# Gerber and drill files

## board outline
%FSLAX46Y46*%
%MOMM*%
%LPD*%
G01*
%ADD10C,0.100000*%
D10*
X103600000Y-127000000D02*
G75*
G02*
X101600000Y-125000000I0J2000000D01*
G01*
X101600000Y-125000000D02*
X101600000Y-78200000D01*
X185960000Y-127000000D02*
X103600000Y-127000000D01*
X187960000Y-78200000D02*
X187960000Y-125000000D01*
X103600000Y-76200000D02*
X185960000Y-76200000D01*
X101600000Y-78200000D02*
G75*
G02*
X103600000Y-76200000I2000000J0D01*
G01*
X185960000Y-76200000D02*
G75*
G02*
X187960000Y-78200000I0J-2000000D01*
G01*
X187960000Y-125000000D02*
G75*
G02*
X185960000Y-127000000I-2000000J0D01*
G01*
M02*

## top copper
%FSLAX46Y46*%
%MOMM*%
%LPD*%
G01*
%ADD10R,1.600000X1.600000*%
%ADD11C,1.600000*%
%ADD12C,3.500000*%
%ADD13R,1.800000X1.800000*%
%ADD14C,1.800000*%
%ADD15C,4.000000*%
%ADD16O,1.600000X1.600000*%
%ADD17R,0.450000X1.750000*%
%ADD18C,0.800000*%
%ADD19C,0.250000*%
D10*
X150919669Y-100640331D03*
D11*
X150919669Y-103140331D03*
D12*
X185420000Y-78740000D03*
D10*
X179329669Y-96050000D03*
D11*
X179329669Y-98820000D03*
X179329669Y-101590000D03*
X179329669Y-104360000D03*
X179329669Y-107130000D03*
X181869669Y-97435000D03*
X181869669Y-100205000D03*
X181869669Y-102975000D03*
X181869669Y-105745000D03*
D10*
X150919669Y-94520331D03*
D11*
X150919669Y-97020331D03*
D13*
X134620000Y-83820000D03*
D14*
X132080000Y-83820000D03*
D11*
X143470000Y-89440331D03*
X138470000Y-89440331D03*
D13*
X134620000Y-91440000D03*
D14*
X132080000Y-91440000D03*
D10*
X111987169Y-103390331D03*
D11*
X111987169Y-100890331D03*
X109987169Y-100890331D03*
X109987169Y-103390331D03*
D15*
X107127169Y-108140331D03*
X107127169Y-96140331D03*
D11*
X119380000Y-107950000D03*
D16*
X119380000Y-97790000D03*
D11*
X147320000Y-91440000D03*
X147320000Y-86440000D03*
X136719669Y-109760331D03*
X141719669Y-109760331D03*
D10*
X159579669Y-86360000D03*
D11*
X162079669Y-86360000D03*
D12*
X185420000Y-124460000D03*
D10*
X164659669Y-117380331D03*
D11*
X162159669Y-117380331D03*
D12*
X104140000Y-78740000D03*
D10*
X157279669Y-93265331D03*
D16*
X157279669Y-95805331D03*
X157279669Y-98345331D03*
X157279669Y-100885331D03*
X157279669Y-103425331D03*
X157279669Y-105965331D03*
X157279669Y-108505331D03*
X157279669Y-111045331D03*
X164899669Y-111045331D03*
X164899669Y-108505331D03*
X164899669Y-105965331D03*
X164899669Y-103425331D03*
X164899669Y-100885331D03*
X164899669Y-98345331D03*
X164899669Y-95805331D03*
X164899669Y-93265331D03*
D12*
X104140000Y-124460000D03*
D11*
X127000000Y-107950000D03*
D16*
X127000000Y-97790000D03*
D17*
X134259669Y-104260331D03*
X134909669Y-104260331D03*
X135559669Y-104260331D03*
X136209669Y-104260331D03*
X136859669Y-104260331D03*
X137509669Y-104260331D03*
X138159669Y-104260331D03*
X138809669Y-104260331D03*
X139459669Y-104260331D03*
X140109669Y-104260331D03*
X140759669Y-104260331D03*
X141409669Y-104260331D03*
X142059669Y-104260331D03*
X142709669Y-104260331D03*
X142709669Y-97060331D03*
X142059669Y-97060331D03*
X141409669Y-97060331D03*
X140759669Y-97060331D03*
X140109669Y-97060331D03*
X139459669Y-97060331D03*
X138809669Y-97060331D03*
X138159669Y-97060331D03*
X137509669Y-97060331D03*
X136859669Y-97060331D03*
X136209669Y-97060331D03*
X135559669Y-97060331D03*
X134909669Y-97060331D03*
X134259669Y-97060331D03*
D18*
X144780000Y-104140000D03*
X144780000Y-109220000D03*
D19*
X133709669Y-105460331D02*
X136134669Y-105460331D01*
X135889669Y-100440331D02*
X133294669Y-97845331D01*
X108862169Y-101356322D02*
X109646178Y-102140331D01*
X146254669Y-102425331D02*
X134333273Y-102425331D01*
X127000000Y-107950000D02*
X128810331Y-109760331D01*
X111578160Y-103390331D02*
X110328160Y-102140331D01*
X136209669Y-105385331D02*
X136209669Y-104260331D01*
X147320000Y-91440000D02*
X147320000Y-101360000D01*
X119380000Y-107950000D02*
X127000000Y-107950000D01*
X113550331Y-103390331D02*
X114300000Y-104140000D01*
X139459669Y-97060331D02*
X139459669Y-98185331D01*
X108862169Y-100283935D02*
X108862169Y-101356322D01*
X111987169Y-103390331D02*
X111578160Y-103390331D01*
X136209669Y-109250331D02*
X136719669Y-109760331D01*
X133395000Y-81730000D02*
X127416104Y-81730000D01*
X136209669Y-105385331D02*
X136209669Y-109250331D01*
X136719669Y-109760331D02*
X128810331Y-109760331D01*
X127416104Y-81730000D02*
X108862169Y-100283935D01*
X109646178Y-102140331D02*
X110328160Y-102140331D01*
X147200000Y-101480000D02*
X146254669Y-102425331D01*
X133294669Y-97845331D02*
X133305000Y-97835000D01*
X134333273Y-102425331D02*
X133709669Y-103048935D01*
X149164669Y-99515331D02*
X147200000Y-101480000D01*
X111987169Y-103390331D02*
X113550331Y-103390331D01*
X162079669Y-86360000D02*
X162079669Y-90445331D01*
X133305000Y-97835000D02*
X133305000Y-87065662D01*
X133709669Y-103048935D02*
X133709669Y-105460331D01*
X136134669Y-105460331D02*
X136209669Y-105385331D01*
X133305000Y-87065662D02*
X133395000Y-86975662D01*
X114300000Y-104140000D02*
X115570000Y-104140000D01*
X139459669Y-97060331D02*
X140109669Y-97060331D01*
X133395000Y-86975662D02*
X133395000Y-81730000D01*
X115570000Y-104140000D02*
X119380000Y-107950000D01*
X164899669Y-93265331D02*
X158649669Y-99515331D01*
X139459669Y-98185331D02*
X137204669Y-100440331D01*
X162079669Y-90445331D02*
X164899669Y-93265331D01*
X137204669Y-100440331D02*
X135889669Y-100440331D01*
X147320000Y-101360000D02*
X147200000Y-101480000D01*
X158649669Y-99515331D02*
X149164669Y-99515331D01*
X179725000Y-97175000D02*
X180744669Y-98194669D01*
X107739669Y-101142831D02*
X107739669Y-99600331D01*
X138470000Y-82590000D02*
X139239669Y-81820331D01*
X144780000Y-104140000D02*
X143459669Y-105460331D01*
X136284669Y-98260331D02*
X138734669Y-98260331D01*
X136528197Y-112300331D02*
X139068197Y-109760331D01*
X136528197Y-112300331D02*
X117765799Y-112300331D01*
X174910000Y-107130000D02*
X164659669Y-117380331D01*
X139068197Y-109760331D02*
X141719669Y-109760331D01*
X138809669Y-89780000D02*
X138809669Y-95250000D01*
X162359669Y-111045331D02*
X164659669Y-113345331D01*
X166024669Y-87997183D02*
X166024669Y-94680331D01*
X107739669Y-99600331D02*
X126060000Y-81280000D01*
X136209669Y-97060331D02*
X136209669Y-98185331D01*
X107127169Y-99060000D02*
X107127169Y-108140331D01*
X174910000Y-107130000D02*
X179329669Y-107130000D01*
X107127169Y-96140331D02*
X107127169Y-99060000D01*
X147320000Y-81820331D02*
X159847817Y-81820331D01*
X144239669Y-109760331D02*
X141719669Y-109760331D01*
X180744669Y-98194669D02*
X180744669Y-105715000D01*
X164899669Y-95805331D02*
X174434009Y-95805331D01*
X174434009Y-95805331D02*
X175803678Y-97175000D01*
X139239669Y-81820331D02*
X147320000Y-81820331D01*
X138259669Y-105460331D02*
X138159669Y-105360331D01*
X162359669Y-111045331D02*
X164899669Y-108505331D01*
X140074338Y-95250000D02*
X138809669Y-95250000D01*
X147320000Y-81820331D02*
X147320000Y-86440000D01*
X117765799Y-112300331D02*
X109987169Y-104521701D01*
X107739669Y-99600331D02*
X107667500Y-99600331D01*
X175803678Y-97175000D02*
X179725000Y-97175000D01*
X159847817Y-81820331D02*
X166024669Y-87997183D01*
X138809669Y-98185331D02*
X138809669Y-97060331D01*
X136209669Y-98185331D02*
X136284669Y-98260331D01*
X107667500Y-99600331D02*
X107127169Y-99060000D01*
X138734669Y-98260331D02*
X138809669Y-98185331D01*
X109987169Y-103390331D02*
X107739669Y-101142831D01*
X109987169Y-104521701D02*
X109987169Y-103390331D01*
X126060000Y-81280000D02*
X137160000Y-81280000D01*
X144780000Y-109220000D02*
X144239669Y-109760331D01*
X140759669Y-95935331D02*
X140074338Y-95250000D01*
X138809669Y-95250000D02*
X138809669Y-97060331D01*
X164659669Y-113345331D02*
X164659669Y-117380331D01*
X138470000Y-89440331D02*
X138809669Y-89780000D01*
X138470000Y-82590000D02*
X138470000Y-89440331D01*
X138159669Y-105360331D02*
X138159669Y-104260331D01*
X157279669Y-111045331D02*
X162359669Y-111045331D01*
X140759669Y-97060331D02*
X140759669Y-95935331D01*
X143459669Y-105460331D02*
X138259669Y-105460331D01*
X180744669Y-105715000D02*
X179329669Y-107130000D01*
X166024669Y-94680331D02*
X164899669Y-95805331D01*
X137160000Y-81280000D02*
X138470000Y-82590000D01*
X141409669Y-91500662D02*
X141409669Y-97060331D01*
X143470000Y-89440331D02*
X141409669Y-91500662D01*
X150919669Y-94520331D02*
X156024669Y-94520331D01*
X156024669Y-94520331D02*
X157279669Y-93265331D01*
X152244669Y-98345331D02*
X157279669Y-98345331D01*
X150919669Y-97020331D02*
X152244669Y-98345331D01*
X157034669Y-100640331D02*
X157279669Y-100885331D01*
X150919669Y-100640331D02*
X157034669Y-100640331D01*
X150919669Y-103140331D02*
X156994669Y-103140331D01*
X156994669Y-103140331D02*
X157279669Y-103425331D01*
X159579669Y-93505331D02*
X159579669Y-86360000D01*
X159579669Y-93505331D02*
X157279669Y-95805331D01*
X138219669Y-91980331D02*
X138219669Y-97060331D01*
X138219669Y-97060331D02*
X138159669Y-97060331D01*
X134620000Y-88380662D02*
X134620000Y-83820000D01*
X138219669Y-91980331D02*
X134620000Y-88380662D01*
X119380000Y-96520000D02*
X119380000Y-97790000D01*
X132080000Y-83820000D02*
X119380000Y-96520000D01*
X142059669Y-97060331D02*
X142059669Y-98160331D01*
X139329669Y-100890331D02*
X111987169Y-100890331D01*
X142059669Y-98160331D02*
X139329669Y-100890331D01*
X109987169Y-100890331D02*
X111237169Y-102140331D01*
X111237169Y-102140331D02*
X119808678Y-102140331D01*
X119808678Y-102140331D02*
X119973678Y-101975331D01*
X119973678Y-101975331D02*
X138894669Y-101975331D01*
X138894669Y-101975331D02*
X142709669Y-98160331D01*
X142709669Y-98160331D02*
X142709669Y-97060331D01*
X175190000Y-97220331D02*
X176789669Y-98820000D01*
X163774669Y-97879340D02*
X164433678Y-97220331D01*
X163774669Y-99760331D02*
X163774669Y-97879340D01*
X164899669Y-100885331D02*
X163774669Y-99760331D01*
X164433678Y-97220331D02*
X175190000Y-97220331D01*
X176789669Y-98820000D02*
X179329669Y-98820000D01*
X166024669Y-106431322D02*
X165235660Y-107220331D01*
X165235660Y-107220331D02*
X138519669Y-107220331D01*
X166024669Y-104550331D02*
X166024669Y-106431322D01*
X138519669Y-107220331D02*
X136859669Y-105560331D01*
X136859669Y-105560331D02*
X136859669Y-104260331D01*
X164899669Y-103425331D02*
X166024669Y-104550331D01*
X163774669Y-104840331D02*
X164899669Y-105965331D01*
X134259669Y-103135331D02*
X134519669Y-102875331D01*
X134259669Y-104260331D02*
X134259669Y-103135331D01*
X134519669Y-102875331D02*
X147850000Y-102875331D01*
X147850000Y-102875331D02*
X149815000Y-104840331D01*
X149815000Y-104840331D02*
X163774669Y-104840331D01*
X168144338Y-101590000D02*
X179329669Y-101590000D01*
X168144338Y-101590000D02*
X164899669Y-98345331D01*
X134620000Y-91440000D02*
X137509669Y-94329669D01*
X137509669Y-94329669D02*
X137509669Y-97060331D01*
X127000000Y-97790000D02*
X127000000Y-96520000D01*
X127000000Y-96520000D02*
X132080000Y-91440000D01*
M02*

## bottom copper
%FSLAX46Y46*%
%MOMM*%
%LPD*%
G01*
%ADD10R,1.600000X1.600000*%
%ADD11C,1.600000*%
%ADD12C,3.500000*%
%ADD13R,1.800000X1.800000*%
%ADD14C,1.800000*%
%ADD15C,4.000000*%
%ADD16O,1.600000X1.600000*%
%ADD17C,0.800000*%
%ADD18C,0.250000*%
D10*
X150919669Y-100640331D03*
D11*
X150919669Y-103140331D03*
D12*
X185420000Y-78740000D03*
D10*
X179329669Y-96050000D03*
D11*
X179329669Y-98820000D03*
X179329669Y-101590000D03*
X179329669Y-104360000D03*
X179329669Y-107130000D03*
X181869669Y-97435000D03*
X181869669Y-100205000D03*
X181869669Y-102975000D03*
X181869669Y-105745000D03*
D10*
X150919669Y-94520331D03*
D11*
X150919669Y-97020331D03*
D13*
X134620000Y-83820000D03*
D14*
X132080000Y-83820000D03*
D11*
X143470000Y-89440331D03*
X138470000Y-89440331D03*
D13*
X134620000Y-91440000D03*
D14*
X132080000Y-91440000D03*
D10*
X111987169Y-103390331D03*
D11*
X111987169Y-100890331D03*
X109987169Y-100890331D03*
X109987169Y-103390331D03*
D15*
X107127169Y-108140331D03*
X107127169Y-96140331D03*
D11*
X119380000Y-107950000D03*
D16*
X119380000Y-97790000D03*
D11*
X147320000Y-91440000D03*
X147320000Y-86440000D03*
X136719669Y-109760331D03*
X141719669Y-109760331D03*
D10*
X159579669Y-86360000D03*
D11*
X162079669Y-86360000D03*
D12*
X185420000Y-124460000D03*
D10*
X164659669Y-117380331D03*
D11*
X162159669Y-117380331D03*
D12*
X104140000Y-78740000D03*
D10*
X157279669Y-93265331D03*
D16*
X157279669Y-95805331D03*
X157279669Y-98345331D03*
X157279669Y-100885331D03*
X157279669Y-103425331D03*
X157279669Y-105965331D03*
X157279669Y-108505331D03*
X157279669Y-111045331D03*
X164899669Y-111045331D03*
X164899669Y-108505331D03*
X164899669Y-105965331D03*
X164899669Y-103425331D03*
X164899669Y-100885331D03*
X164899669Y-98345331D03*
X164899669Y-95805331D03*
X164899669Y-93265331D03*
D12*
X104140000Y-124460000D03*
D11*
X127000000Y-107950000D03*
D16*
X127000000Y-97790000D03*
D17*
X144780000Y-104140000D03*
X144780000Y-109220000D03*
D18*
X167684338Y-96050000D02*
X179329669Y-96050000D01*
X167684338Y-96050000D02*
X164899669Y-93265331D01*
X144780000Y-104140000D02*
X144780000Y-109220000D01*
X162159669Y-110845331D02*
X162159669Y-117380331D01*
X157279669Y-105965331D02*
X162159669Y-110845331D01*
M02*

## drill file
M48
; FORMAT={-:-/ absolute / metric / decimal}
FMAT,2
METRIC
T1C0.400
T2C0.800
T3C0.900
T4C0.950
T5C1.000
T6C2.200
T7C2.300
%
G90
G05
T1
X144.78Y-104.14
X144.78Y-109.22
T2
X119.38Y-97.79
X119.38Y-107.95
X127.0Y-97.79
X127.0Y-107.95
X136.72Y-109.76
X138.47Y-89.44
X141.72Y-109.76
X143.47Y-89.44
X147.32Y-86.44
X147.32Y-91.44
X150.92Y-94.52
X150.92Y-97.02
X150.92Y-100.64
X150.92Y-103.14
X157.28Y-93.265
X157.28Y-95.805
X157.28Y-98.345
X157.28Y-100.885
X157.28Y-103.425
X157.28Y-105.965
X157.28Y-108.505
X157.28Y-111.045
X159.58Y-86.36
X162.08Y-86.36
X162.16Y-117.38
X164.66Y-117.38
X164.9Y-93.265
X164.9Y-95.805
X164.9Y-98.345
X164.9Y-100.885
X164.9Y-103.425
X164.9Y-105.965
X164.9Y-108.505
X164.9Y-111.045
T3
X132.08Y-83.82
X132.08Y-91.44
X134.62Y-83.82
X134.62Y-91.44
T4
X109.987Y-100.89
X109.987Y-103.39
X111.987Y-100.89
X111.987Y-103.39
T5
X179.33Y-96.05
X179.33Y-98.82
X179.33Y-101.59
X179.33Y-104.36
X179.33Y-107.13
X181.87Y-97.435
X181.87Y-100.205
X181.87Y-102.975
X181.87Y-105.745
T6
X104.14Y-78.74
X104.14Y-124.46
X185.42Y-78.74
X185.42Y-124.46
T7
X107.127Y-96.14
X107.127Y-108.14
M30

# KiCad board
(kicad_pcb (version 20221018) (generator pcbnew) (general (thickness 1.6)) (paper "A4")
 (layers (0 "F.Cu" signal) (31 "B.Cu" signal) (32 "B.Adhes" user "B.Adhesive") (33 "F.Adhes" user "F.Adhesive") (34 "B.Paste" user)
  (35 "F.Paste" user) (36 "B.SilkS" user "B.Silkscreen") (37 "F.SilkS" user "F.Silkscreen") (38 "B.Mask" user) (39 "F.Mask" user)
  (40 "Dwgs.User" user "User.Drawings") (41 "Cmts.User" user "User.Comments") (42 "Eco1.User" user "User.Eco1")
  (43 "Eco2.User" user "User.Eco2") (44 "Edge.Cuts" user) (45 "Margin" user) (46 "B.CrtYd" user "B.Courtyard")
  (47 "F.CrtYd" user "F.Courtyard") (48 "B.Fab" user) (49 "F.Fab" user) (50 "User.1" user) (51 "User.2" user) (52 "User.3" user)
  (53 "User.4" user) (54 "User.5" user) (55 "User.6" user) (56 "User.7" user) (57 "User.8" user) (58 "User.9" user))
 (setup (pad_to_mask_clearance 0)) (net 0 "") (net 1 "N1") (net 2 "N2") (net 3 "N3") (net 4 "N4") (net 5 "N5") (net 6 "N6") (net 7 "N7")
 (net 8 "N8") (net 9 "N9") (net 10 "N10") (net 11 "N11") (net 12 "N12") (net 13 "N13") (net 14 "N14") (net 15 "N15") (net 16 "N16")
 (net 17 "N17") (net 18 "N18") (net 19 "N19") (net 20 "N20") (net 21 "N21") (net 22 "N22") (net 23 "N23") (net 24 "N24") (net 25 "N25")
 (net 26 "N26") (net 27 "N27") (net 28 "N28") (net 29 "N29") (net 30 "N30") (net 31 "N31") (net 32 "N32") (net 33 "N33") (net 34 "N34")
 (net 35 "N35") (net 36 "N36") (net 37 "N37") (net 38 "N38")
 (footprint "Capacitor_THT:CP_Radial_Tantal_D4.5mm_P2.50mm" (layer "F.Cu") (at 150.919669 100.640331 -90)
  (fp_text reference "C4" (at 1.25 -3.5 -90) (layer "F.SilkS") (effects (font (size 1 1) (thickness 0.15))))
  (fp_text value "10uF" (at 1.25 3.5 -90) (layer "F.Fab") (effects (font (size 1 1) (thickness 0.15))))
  (pad "1" thru_hole rect (at 0 0 270) (size 1.6 1.6) (drill 0.8) (layers "*.Cu" "*.Mask") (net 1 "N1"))
  (pad "2" thru_hole circle (at 2.5 0 270) (size 1.6 1.6) (drill 0.8) (layers "*.Cu" "*.Mask") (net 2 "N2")))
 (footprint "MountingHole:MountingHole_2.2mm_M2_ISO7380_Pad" (layer "F.Cu") (at 185.42 78.74)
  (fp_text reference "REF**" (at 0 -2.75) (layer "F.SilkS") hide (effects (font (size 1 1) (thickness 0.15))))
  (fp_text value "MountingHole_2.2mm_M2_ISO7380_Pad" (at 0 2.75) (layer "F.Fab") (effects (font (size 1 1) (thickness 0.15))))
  (pad "1" thru_hole circle (at 0 0) (size 3.5 3.5) (drill 2.2) (layers "*.Cu" "*.Mask")))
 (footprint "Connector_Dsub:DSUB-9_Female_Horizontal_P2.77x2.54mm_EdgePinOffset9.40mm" (layer "F.Cu") (at 179.329669 96.05 90)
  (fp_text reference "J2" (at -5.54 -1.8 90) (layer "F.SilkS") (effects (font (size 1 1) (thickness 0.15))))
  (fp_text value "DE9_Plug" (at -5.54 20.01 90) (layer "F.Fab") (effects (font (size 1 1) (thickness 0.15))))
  (pad "1" thru_hole rect (at 0 0 90) (size 1.6 1.6) (drill 1) (layers "*.Cu" "*.Mask") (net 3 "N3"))
  (pad "2" thru_hole circle (at -2.77 0 90) (size 1.6 1.6) (drill 1) (layers "*.Cu" "*.Mask") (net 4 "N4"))
  (pad "3" thru_hole circle (at -5.54 0 90) (size 1.6 1.6) (drill 1) (layers "*.Cu" "*.Mask") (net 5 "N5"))
  (pad "4" thru_hole circle (at -8.31 0 90) (size 1.6 1.6) (drill 1) (layers "*.Cu" "*.Mask") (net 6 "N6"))
  (pad "5" thru_hole circle (at -11.08 0 90) (size 1.6 1.6) (drill 1) (layers "*.Cu" "*.Mask") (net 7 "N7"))
  (pad "6" thru_hole circle (at -1.385 2.54 90) (size 1.6 1.6) (drill 1) (layers "*.Cu" "*.Mask") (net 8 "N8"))
  (pad "7" thru_hole circle (at -4.155 2.54 90) (size 1.6 1.6) (drill 1) (layers "*.Cu" "*.Mask") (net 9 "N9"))
  (pad "8" thru_hole circle (at -6.925 2.54 90) (size 1.6 1.6) (drill 1) (layers "*.Cu" "*.Mask") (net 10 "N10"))
  (pad "9" thru_hole circle (at -9.695 2.54 90) (size 1.6 1.6) (drill 1) (layers "*.Cu" "*.Mask") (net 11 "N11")))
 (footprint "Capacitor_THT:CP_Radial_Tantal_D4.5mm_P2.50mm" (layer "F.Cu") (at 150.919669 94.520331 -90)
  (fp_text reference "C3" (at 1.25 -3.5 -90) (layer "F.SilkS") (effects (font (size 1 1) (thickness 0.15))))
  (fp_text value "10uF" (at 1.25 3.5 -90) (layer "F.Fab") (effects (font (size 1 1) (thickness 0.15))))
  (pad "1" thru_hole rect (at 0 0 270) (size 1.6 1.6) (drill 0.8) (layers "*.Cu" "*.Mask") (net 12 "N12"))
  (pad "2" thru_hole circle (at 2.5 0 270) (size 1.6 1.6) (drill 0.8) (layers "*.Cu" "*.Mask") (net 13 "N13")))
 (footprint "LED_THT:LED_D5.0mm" (layer "F.Cu") (at 134.62 83.82 180)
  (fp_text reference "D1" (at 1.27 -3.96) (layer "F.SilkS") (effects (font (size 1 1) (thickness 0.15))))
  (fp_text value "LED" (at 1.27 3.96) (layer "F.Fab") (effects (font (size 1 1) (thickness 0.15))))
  (pad "1" thru_hole rect (at 0 0 180) (size 1.8 1.8) (drill 0.9) (layers "*.Cu" "*.Mask") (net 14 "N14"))
  (pad "2" thru_hole circle (at 2.54 0 180) (size 1.8 1.8) (drill 0.9) (layers "*.Cu" "*.Mask") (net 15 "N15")))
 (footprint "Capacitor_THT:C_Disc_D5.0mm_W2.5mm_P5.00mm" (layer "F.Cu") (at 143.47 89.440331 180)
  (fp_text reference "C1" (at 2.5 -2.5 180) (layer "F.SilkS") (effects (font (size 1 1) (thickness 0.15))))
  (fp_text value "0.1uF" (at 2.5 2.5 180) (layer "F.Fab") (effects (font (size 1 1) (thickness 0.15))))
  (pad "1" thru_hole circle (at 0 0 180) (size 1.6 1.6) (drill 0.8) (layers "*.Cu" "*.Mask") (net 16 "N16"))
  (pad "2" thru_hole circle (at 5 0 180) (size 1.6 1.6) (drill 0.8) (layers "*.Cu" "*.Mask") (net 7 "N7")))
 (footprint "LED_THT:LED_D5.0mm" (layer "F.Cu") (at 134.62 91.44 180)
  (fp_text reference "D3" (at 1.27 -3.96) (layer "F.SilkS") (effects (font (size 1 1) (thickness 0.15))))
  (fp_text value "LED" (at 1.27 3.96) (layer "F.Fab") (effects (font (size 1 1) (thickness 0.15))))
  (pad "1" thru_hole rect (at 0 0 180) (size 1.8 1.8) (drill 0.9) (layers "*.Cu" "*.Mask") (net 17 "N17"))
  (pad "2" thru_hole circle (at 2.54 0 180) (size 1.8 1.8) (drill 0.9) (layers "*.Cu" "*.Mask") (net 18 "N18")))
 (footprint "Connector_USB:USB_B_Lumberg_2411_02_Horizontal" (layer "F.Cu") (at 111.987169 103.390331 180)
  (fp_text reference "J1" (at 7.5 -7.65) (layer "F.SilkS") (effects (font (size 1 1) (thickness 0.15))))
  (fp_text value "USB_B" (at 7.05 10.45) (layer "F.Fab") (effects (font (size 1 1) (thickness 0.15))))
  (pad "1" thru_hole rect (at 0 0 270) (size 1.6 1.6) (drill 0.95) (layers "*.Cu" "*.Mask") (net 3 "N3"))
  (pad "2" thru_hole circle (at 0 2.5 270) (size 1.6 1.6) (drill 0.95) (layers "*.Cu" "*.Mask") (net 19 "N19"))
  (pad "3" thru_hole circle (at 2 2.5 270) (size 1.6 1.6) (drill 0.95) (layers "*.Cu" "*.Mask") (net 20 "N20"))
  (pad "4" thru_hole circle (at 2 0 270) (size 1.6 1.6) (drill 0.95) (layers "*.Cu" "*.Mask") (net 7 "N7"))
  (pad "5" thru_hole circle (at 4.86 -4.75 270) (size 4 4) (drill 2.3) (layers "*.Cu" "*.Mask") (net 7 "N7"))
  (pad "5" thru_hole circle (at 4.86 7.25 270) (size 4 4) (drill 2.3) (layers "*.Cu" "*.Mask") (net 7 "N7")))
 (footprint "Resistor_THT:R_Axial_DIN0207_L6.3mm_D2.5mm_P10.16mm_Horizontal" (layer "F.Cu") (at 119.38 107.95 90)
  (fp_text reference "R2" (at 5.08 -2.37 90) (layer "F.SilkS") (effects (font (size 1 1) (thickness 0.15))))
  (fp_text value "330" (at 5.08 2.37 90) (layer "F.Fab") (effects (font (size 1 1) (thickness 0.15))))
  (pad "1" thru_hole circle (at 0 0 90) (size 1.6 1.6) (drill 0.8) (layers "*.Cu" "*.Mask") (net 3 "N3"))
  (pad "2" thru_hole oval (at 10.16 0 90) (size 1.6 1.6) (drill 0.8) (layers "*.Cu" "*.Mask") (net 15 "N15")))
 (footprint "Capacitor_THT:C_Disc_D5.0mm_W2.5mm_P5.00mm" (layer "F.Cu") (at 147.32 91.44 90)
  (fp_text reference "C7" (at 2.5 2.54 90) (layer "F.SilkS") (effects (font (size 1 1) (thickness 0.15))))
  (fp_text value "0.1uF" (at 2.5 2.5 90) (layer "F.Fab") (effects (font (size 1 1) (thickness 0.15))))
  (pad "1" thru_hole circle (at 0 0 90) (size 1.6 1.6) (drill 0.8) (layers "*.Cu" "*.Mask") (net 3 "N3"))
  (pad "2" thru_hole circle (at 5 0 90) (size 1.6 1.6) (drill 0.8) (layers "*.Cu" "*.Mask") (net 7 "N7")))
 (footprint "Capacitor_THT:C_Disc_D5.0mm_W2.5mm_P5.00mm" (layer "F.Cu") (at 136.719669 109.760331)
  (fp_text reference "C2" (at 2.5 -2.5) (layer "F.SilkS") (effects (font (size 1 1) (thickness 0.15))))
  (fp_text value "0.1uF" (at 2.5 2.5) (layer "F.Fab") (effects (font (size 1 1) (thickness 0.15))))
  (pad "1" thru_hole circle (at 0 0) (size 1.6 1.6) (drill 0.8) (layers "*.Cu" "*.Mask") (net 3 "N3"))
  (pad "2" thru_hole circle (at 5 0) (size 1.6 1.6) (drill 0.8) (layers "*.Cu" "*.Mask") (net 7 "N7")))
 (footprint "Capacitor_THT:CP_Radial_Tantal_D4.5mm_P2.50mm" (layer "F.Cu") (at 159.579669 86.36)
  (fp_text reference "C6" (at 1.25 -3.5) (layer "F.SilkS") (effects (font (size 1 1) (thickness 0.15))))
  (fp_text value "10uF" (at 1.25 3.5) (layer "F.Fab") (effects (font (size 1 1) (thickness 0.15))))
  (pad "1" thru_hole rect (at 0 0) (size 1.6 1.6) (drill 0.8) (layers "*.Cu" "*.Mask") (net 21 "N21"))
  (pad "2" thru_hole circle (at 2.5 0) (size 1.6 1.6) (drill 0.8) (layers "*.Cu" "*.Mask") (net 3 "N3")))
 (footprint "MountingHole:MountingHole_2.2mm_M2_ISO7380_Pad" (layer "F.Cu") (at 185.42 124.46)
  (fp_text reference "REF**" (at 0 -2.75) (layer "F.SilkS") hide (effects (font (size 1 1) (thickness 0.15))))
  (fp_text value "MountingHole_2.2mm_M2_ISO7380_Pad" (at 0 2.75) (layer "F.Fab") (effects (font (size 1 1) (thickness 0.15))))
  (pad "1" thru_hole circle (at 0 0) (size 3.5 3.5) (drill 2.2) (layers "*.Cu" "*.Mask")))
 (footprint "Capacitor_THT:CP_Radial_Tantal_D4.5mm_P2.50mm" (layer "F.Cu") (at 164.659669 117.380331 180)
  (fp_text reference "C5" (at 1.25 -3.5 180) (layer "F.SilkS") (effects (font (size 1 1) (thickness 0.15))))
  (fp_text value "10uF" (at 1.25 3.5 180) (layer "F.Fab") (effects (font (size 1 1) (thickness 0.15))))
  (pad "1" thru_hole rect (at 0 0 180) (size 1.6 1.6) (drill 0.8) (layers "*.Cu" "*.Mask") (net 7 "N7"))
  (pad "2" thru_hole circle (at 2.5 0 180) (size 1.6 1.6) (drill 0.8) (layers "*.Cu" "*.Mask") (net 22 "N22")))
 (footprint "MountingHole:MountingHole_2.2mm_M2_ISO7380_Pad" (layer "F.Cu") (at 104.14 78.74)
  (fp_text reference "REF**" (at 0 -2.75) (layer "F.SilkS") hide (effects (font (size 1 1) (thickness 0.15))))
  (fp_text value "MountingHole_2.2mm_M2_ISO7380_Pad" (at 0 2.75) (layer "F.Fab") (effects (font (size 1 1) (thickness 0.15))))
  (pad "1" thru_hole circle (at 0 0) (size 3.5 3.5) (drill 2.2) (layers "*.Cu" "*.Mask")))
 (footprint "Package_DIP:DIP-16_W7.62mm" (layer "F.Cu") (at 157.279669 93.265331)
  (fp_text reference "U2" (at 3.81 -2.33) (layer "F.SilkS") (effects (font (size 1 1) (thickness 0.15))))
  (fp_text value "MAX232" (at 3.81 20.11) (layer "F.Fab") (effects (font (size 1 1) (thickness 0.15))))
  (pad "1" thru_hole rect (at 0 0) (size 1.6 1.6) (drill 0.8) (layers "*.Cu" "*.Mask") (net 12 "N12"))
  (pad "2" thru_hole oval (at 0 2.54) (size 1.6 1.6) (drill 0.8) (layers "*.Cu" "*.Mask") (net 21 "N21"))
  (pad "3" thru_hole oval (at 0 5.08) (size 1.6 1.6) (drill 0.8) (layers "*.Cu" "*.Mask") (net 13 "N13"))
  (pad "4" thru_hole oval (at 0 7.62) (size 1.6 1.6) (drill 0.8) (layers "*.Cu" "*.Mask") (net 1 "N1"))
  (pad "5" thru_hole oval (at 0 10.16) (size 1.6 1.6) (drill 0.8) (layers "*.Cu" "*.Mask") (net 2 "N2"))
  (pad "6" thru_hole oval (at 0 12.7) (size 1.6 1.6) (drill 0.8) (layers "*.Cu" "*.Mask") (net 22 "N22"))
  (pad "7" thru_hole oval (at 0 15.24) (size 1.6 1.6) (drill 0.8) (layers "*.Cu" "*.Mask") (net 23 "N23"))
  (pad "8" thru_hole oval (at 0 17.78) (size 1.6 1.6) (drill 0.8) (layers "*.Cu" "*.Mask") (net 7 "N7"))
  (pad "9" thru_hole oval (at 7.62 17.78) (size 1.6 1.6) (drill 0.8) (layers "*.Cu" "*.Mask") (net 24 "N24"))
  (pad "10" thru_hole oval (at 7.62 15.24) (size 1.6 1.6) (drill 0.8) (layers "*.Cu" "*.Mask") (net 7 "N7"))
  (pad "11" thru_hole oval (at 7.62 12.7) (size 1.6 1.6) (drill 0.8) (layers "*.Cu" "*.Mask") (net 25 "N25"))
  (pad "12" thru_hole oval (at 7.62 10.16) (size 1.6 1.6) (drill 0.8) (layers "*.Cu" "*.Mask") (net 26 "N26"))
  (pad "13" thru_hole oval (at 7.62 7.62) (size 1.6 1.6) (drill 0.8) (layers "*.Cu" "*.Mask") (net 4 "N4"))
  (pad "14" thru_hole oval (at 7.62 5.08) (size 1.6 1.6) (drill 0.8) (layers "*.Cu" "*.Mask") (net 5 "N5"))
  (pad "15" thru_hole oval (at 7.62 2.54) (size 1.6 1.6) (drill 0.8) (layers "*.Cu" "*.Mask") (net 7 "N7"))
  (pad "16" thru_hole oval (at 7.62 0) (size 1.6 1.6) (drill 0.8) (layers "*.Cu" "*.Mask") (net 3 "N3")))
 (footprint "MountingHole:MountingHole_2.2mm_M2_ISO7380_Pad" (layer "F.Cu") (at 104.14 124.46)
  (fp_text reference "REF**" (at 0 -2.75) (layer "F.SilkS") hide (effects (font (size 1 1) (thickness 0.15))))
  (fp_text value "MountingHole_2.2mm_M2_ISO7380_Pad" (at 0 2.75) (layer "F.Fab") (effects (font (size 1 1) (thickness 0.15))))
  (pad "1" thru_hole circle (at 0 0) (size 3.5 3.5) (drill 2.2) (layers "*.Cu" "*.Mask")))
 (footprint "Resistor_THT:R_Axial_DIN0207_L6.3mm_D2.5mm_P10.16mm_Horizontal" (layer "F.Cu") (at 127 107.95 90)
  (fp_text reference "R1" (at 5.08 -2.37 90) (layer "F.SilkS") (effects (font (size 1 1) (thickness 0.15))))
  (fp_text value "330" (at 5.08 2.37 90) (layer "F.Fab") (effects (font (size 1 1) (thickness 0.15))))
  (pad "1" thru_hole circle (at 0 0 90) (size 1.6 1.6) (drill 0.8) (layers "*.Cu" "*.Mask") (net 3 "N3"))
  (pad "2" thru_hole oval (at 10.16 0 90) (size 1.6 1.6) (drill 0.8) (layers "*.Cu" "*.Mask") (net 18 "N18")))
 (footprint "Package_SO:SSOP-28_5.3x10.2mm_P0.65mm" (layer "F.Cu") (at 138.484669 100.660331 90)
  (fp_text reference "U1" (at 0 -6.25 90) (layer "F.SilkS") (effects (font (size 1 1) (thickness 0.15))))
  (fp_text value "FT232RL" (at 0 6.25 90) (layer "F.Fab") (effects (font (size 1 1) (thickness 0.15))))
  (pad "1" smd rect (at -3.6 -4.225 90) (size 1.75 0.45) (layers "F.Cu" "F.Paste" "F.Mask") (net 25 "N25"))
  (pad "2" smd rect (at -3.6 -3.575 90) (size 1.75 0.45) (layers "F.Cu" "F.Paste" "F.Mask") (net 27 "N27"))
  (pad "3" smd rect (at -3.6 -2.925 90) (size 1.75 0.45) (layers "F.Cu" "F.Paste" "F.Mask") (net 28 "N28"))
  (pad "4" smd rect (at -3.6 -2.275 90) (size 1.75 0.45) (layers "F.Cu" "F.Paste" "F.Mask") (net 3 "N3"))
  (pad "5" smd rect (at -3.6 -1.625 90) (size 1.75 0.45) (layers "F.Cu" "F.Paste" "F.Mask") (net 26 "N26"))
  (pad "6" smd rect (at -3.6 -0.975 90) (size 1.75 0.45) (layers "F.Cu" "F.Paste" "F.Mask") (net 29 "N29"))
  (pad "7" smd rect (at -3.6 -0.325 90) (size 1.75 0.45) (layers "F.Cu" "F.Paste" "F.Mask") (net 7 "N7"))
  (pad "8" smd rect (at -3.6 0.325 90) (size 1.75 0.45) (layers "F.Cu" "F.Paste" "F.Mask"))
  (pad "9" smd rect (at -3.6 0.975 90) (size 1.75 0.45) (layers "F.Cu" "F.Paste" "F.Mask") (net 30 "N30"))
  (pad "10" smd rect (at -3.6 1.625 90) (size 1.75 0.45) (layers "F.Cu" "F.Paste" "F.Mask") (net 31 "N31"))
  (pad "11" smd rect (at -3.6 2.275 90) (size 1.75 0.45) (layers "F.Cu" "F.Paste" "F.Mask") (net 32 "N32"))
  (pad "12" smd rect (at -3.6 2.925 90) (size 1.75 0.45) (layers "F.Cu" "F.Paste" "F.Mask") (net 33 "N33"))
  (pad "13" smd rect (at -3.6 3.575 90) (size 1.75 0.45) (layers "F.Cu" "F.Paste" "F.Mask") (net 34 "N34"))
  (pad "14" smd rect (at -3.6 4.225 90) (size 1.75 0.45) (layers "F.Cu" "F.Paste" "F.Mask") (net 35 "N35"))
  (pad "15" smd rect (at 3.6 4.225 90) (size 1.75 0.45) (layers "F.Cu" "F.Paste" "F.Mask") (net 20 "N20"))
  (pad "16" smd rect (at 3.6 3.575 90) (size 1.75 0.45) (layers "F.Cu" "F.Paste" "F.Mask") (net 19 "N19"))
  (pad "17" smd rect (at 3.6 2.925 90) (size 1.75 0.45) (layers "F.Cu" "F.Paste" "F.Mask") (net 16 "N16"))
  (pad "18" smd rect (at 3.6 2.275 90) (size 1.75 0.45) (layers "F.Cu" "F.Paste" "F.Mask") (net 7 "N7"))
  (pad "19" smd rect (at 3.6 1.625 90) (size 1.75 0.45) (layers "F.Cu" "F.Paste" "F.Mask") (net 3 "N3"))
  (pad "20" smd rect (at 3.6 0.975 90) (size 1.75 0.45) (layers "F.Cu" "F.Paste" "F.Mask") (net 3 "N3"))
  (pad "21" smd rect (at 3.6 0.325 90) (size 1.75 0.45) (layers "F.Cu" "F.Paste" "F.Mask") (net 7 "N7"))
  (pad "22" smd rect (at 3.6 -0.325 90) (size 1.75 0.45) (layers "F.Cu" "F.Paste" "F.Mask") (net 14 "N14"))
  (pad "23" smd rect (at 3.6 -0.975 90) (size 1.75 0.45) (layers "F.Cu" "F.Paste" "F.Mask") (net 17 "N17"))
  (pad "24" smd rect (at 3.6 -1.625 90) (size 1.75 0.45) (layers "F.Cu" "F.Paste" "F.Mask"))
  (pad "25" smd rect (at 3.6 -2.275 90) (size 1.75 0.45) (layers "F.Cu" "F.Paste" "F.Mask") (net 7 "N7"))
  (pad "26" smd rect (at 3.6 -2.925 90) (size 1.75 0.45) (layers "F.Cu" "F.Paste" "F.Mask") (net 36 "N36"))
  (pad "27" smd rect (at 3.6 -3.575 90) (size 1.75 0.45) (layers "F.Cu" "F.Paste" "F.Mask") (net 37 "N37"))
  (pad "28" smd rect (at 3.6 -4.225 90) (size 1.75 0.45) (layers "F.Cu" "F.Paste" "F.Mask") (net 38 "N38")))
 (gr_arc (start 103.6 127) (mid 102.185786 126.414214) (end 101.6 125) (stroke (width 0.1) (type default)) (layer "Edge.Cuts"))
 (gr_line (start 101.6 125) (end 101.6 78.2) (stroke (width 0.1) (type default)) (layer "Edge.Cuts"))
 (gr_line (start 185.96 127) (end 103.6 127) (stroke (width 0.1) (type default)) (layer "Edge.Cuts"))
 (gr_line (start 187.96 78.2) (end 187.96 125) (stroke (width 0.1) (type default)) (layer "Edge.Cuts"))
 (gr_line (start 103.6 76.2) (end 185.96 76.2) (stroke (width 0.1) (type default)) (layer "Edge.Cuts"))
 (gr_arc (start 101.6 78.2) (mid 102.185786 76.785786) (end 103.6 76.2) (stroke (width 0.1) (type default)) (layer "Edge.Cuts"))
 (gr_arc (start 185.96 76.2) (mid 187.374214 76.785786) (end 187.96 78.2) (stroke (width 0.1) (type default)) (layer "Edge.Cuts"))
 (gr_arc (start 187.96 125) (mid 187.374214 126.414214) (end 185.96 127) (stroke (width 0.1) (type default)) (layer "Edge.Cuts"))
 (segment (start 133.709669 105.460331) (end 136.134669 105.460331) (width 0.25) (layer "F.Cu") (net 3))
 (segment (start 135.889669 100.440331) (end 133.294669 97.845331) (width 0.25) (layer "F.Cu") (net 3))
 (segment (start 108.862169 101.356322) (end 109.646178 102.140331) (width 0.25) (layer "F.Cu") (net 3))
 (segment (start 146.254669 102.425331) (end 134.333273 102.425331) (width 0.25) (layer "F.Cu") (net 3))
 (segment (start 127 107.95) (end 128.810331 109.760331) (width 0.25) (layer "F.Cu") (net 3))
 (segment (start 111.57816 103.390331) (end 110.32816 102.140331) (width 0.25) (layer "F.Cu") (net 3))
 (segment (start 136.209669 105.385331) (end 136.209669 104.260331) (width 0.25) (layer "F.Cu") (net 3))
 (segment (start 147.32 91.44) (end 147.32 101.36) (width 0.25) (layer "F.Cu") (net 3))
 (segment (start 119.38 107.95) (end 127 107.95) (width 0.25) (layer "F.Cu") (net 3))
 (segment (start 113.550331 103.390331) (end 114.3 104.14) (width 0.25) (layer "F.Cu") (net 3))
 (segment (start 139.459669 97.060331) (end 139.459669 98.185331) (width 0.25) (layer "F.Cu") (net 3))
 (segment (start 108.862169 100.283935) (end 108.862169 101.356322) (width 0.25) (layer "F.Cu") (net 3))
 (segment (start 111.987169 103.390331) (end 111.57816 103.390331) (width 0.25) (layer "F.Cu") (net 3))
 (segment (start 136.209669 109.250331) (end 136.719669 109.760331) (width 0.25) (layer "F.Cu") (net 3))
 (segment (start 133.395 81.73) (end 127.416104 81.73) (width 0.25) (layer "F.Cu") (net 3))
 (segment (start 136.209669 105.385331) (end 136.209669 109.250331) (width 0.25) (layer "F.Cu") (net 3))
 (segment (start 136.719669 109.760331) (end 128.810331 109.760331) (width 0.25) (layer "F.Cu") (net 3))
 (segment (start 127.416104 81.73) (end 108.862169 100.283935) (width 0.25) (layer "F.Cu") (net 3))
 (segment (start 109.646178 102.140331) (end 110.32816 102.140331) (width 0.25) (layer "F.Cu") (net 3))
 (segment (start 147.2 101.48) (end 146.254669 102.425331) (width 0.25) (layer "F.Cu") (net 3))
 (segment (start 133.294669 97.845331) (end 133.305 97.835) (width 0.25) (layer "F.Cu") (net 3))
 (segment (start 134.333273 102.425331) (end 133.709669 103.048935) (width 0.25) (layer "F.Cu") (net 3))
 (segment (start 149.164669 99.515331) (end 147.2 101.48) (width 0.25) (layer "F.Cu") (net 3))
 (segment (start 111.987169 103.390331) (end 113.550331 103.390331) (width 0.25) (layer "F.Cu") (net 3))
 (segment (start 162.079669 86.36) (end 162.079669 90.445331) (width 0.25) (layer "F.Cu") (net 3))
 (segment (start 133.305 97.835) (end 133.305 87.065662) (width 0.25) (layer "F.Cu") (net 3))
 (segment (start 133.709669 103.048935) (end 133.709669 105.460331) (width 0.25) (layer "F.Cu") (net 3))
 (segment (start 136.134669 105.460331) (end 136.209669 105.385331) (width 0.25) (layer "F.Cu") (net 3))
 (segment (start 133.305 87.065662) (end 133.395 86.975662) (width 0.25) (layer "F.Cu") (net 3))
 (segment (start 114.3 104.14) (end 115.57 104.14) (width 0.25) (layer "F.Cu") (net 3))
 (segment (start 139.459669 97.060331) (end 140.109669 97.060331) (width 0.25) (layer "F.Cu") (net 3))
 (segment (start 133.395 86.975662) (end 133.395 81.73) (width 0.25) (layer "F.Cu") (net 3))
 (segment (start 115.57 104.14) (end 119.38 107.95) (width 0.25) (layer "F.Cu") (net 3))
 (segment (start 164.899669 93.265331) (end 158.649669 99.515331) (width 0.25) (layer "F.Cu") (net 3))
 (segment (start 139.459669 98.185331) (end 137.204669 100.440331) (width 0.25) (layer "F.Cu") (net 3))
 (segment (start 162.079669 90.445331) (end 164.899669 93.265331) (width 0.25) (layer "F.Cu") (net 3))
 (segment (start 137.204669 100.440331) (end 135.889669 100.440331) (width 0.25) (layer "F.Cu") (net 3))
 (segment (start 147.32 101.36) (end 147.2 101.48) (width 0.25) (layer "F.Cu") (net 3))
 (segment (start 158.649669 99.515331) (end 149.164669 99.515331) (width 0.25) (layer "F.Cu") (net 3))
 (segment (start 167.684338 96.05) (end 179.329669 96.05) (width 0.25) (layer "B.Cu") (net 3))
 (segment (start 167.684338 96.05) (end 164.899669 93.265331) (width 0.25) (layer "B.Cu") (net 3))
 (segment (start 179.725 97.175) (end 180.744669 98.194669) (width 0.25) (layer "F.Cu") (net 7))
 (segment (start 107.739669 101.142831) (end 107.739669 99.600331) (width 0.25) (layer "F.Cu") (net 7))
 (segment (start 138.47 82.59) (end 139.239669 81.820331) (width 0.25) (layer "F.Cu") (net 7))
 (segment (start 144.78 104.14) (end 143.459669 105.460331) (width 0.25) (layer "F.Cu") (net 7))
 (segment (start 136.284669 98.260331) (end 138.734669 98.260331) (width 0.25) (layer "F.Cu") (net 7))
 (segment (start 136.528197 112.300331) (end 139.068197 109.760331) (width 0.25) (layer "F.Cu") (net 7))
 (segment (start 136.528197 112.300331) (end 117.765799 112.300331) (width 0.25) (layer "F.Cu") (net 7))
 (segment (start 174.91 107.13) (end 164.659669 117.380331) (width 0.25) (layer "F.Cu") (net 7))
 (segment (start 139.068197 109.760331) (end 141.719669 109.760331) (width 0.25) (layer "F.Cu") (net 7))
 (segment (start 138.809669 89.78) (end 138.809669 95.25) (width 0.25) (layer "F.Cu") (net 7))
 (segment (start 162.359669 111.045331) (end 164.659669 113.345331) (width 0.25) (layer "F.Cu") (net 7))
 (segment (start 166.024669 87.997183) (end 166.024669 94.680331) (width 0.25) (layer "F.Cu") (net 7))
 (segment (start 107.739669 99.600331) (end 126.06 81.28) (width 0.25) (layer "F.Cu") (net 7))
 (segment (start 136.209669 97.060331) (end 136.209669 98.185331) (width 0.25) (layer "F.Cu") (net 7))
 (segment (start 107.127169 99.06) (end 107.127169 108.140331) (width 0.25) (layer "F.Cu") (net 7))
 (segment (start 174.91 107.13) (end 179.329669 107.13) (width 0.25) (layer "F.Cu") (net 7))
 (segment (start 107.127169 96.140331) (end 107.127169 99.06) (width 0.25) (layer "F.Cu") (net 7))
 (segment (start 147.32 81.820331) (end 159.847817 81.820331) (width 0.25) (layer "F.Cu") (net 7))
 (segment (start 144.239669 109.760331) (end 141.719669 109.760331) (width 0.25) (layer "F.Cu") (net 7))
 (segment (start 180.744669 98.194669) (end 180.744669 105.715) (width 0.25) (layer "F.Cu") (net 7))
 (segment (start 164.899669 95.805331) (end 174.434009 95.805331) (width 0.25) (layer "F.Cu") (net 7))
 (segment (start 174.434009 95.805331) (end 175.803678 97.175) (width 0.25) (layer "F.Cu") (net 7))
 (segment (start 139.239669 81.820331) (end 147.32 81.820331) (width 0.25) (layer "F.Cu") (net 7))
 (segment (start 138.259669 105.460331) (end 138.159669 105.360331) (width 0.25) (layer "F.Cu") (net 7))
 (segment (start 162.359669 111.045331) (end 164.899669 108.505331) (width 0.25) (layer "F.Cu") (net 7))
 (segment (start 140.074338 95.25) (end 138.809669 95.25) (width 0.25) (layer "F.Cu") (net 7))
 (segment (start 147.32 81.820331) (end 147.32 86.44) (width 0.25) (layer "F.Cu") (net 7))
 (segment (start 117.765799 112.300331) (end 109.987169 104.521701) (width 0.25) (layer "F.Cu") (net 7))
 (segment (start 107.739669 99.600331) (end 107.6675 99.600331) (width 0.25) (layer "F.Cu") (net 7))
 (segment (start 175.803678 97.175) (end 179.725 97.175) (width 0.25) (layer "F.Cu") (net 7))
 (segment (start 159.847817 81.820331) (end 166.024669 87.997183) (width 0.25) (layer "F.Cu") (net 7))
 (segment (start 138.809669 98.185331) (end 138.809669 97.060331) (width 0.25) (layer "F.Cu") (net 7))
 (segment (start 136.209669 98.185331) (end 136.284669 98.260331) (width 0.25) (layer "F.Cu") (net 7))
 (segment (start 107.6675 99.600331) (end 107.127169 99.06) (width 0.25) (layer "F.Cu") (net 7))
 (segment (start 138.734669 98.260331) (end 138.809669 98.185331) (width 0.25) (layer "F.Cu") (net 7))
 (segment (start 109.987169 103.390331) (end 107.739669 101.142831) (width 0.25) (layer "F.Cu") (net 7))
 (segment (start 109.987169 104.521701) (end 109.987169 103.390331) (width 0.25) (layer "F.Cu") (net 7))
 (segment (start 126.06 81.28) (end 137.16 81.28) (width 0.25) (layer "F.Cu") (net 7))
 (segment (start 144.78 109.22) (end 144.239669 109.760331) (width 0.25) (layer "F.Cu") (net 7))
 (segment (start 140.759669 95.935331) (end 140.074338 95.25) (width 0.25) (layer "F.Cu") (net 7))
 (segment (start 138.809669 95.25) (end 138.809669 97.060331) (width 0.25) (layer "F.Cu") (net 7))
 (segment (start 164.659669 113.345331) (end 164.659669 117.380331) (width 0.25) (layer "F.Cu") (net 7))
 (segment (start 138.47 89.440331) (end 138.809669 89.78) (width 0.25) (layer "F.Cu") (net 7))
 (segment (start 138.47 82.59) (end 138.47 89.440331) (width 0.25) (layer "F.Cu") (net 7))
 (segment (start 138.159669 105.360331) (end 138.159669 104.260331) (width 0.25) (layer "F.Cu") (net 7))
 (segment (start 157.279669 111.045331) (end 162.359669 111.045331) (width 0.25) (layer "F.Cu") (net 7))
 (segment (start 140.759669 97.060331) (end 140.759669 95.935331) (width 0.25) (layer "F.Cu") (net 7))
 (segment (start 143.459669 105.460331) (end 138.259669 105.460331) (width 0.25) (layer "F.Cu") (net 7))
 (segment (start 180.744669 105.715) (end 179.329669 107.13) (width 0.25) (layer "F.Cu") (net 7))
 (segment (start 166.024669 94.680331) (end 164.899669 95.805331) (width 0.25) (layer "F.Cu") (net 7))
 (segment (start 137.16 81.28) (end 138.47 82.59) (width 0.25) (layer "F.Cu") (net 7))
 (via (at 144.78 104.14) (size 0.8) (drill 0.4) (layers "F.Cu" "B.Cu") (free) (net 7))
 (via (at 144.78 109.22) (size 0.8) (drill 0.4) (layers "F.Cu" "B.Cu") (free) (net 7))
 (segment (start 144.78 104.14) (end 144.78 109.22) (width 0.25) (layer "B.Cu") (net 7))
 (segment (start 141.409669 91.500662) (end 141.409669 97.060331) (width 0.25) (layer "F.Cu") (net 16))
 (segment (start 143.47 89.440331) (end 141.409669 91.500662) (width 0.25) (layer "F.Cu") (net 16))
 (segment (start 150.919669 94.520331) (end 156.024669 94.520331) (width 0.25) (layer "F.Cu") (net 12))
 (segment (start 156.024669 94.520331) (end 157.279669 93.265331) (width 0.25) (layer "F.Cu") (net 12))
 (segment (start 152.244669 98.345331) (end 157.279669 98.345331) (width 0.25) (layer "F.Cu") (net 13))
 (segment (start 150.919669 97.020331) (end 152.244669 98.345331) (width 0.25) (layer "F.Cu") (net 13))
 (segment (start 157.034669 100.640331) (end 157.279669 100.885331) (width 0.25) (layer "F.Cu") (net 1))
 (segment (start 150.919669 100.640331) (end 157.034669 100.640331) (width 0.25) (layer "F.Cu") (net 1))
 (segment (start 150.919669 103.140331) (end 156.994669 103.140331) (width 0.25) (layer "F.Cu") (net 2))
 (segment (start 156.994669 103.140331) (end 157.279669 103.425331) (width 0.25) (layer "F.Cu") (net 2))
 (segment (start 162.159669 110.845331) (end 162.159669 117.380331) (width 0.25) (layer "B.Cu") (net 22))
 (segment (start 157.279669 105.965331) (end 162.159669 110.845331) (width 0.25) (layer "B.Cu") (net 22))
 (segment (start 159.579669 93.505331) (end 159.579669 86.36) (width 0.25) (layer "F.Cu") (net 21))
 (segment (start 159.579669 93.505331) (end 157.279669 95.805331) (width 0.25) (layer "F.Cu") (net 21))
 (segment (start 138.219669 91.980331) (end 138.219669 97.060331) (width 0.25) (layer "F.Cu") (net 14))
 (segment (start 138.219669 97.060331) (end 138.159669 97.060331) (width 0.25) (layer "F.Cu") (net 14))
 (segment (start 134.62 88.380662) (end 134.62 83.82) (width 0.25) (layer "F.Cu") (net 14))
 (segment (start 138.219669 91.980331) (end 134.62 88.380662) (width 0.25) (layer "F.Cu") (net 14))
 (segment (start 119.38 96.52) (end 119.38 97.79) (width 0.25) (layer "F.Cu") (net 15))
 (segment (start 132.08 83.82) (end 119.38 96.52) (width 0.25) (layer "F.Cu") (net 15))
 (segment (start 142.059669 97.060331) (end 142.059669 98.160331) (width 0.25) (layer "F.Cu") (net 19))
 (segment (start 139.329669 100.890331) (end 111.987169 100.890331) (width 0.25) (layer "F.Cu") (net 19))
 (segment (start 142.059669 98.160331) (end 139.329669 100.890331) (width 0.25) (layer "F.Cu") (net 19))
 (segment (start 109.987169 100.890331) (end 111.237169 102.140331) (width 0.25) (layer "F.Cu") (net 20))
 (segment (start 111.237169 102.140331) (end 119.808678 102.140331) (width 0.25) (layer "F.Cu") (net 20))
 (segment (start 119.808678 102.140331) (end 119.973678 101.975331) (width 0.25) (layer "F.Cu") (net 20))
 (segment (start 119.973678 101.975331) (end 138.894669 101.975331) (width 0.25) (layer "F.Cu") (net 20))
 (segment (start 138.894669 101.975331) (end 142.709669 98.160331) (width 0.25) (layer "F.Cu") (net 20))
 (segment (start 142.709669 98.160331) (end 142.709669 97.060331) (width 0.25) (layer "F.Cu") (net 20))
 (segment (start 175.19 97.220331) (end 176.789669 98.82) (width 0.25) (layer "F.Cu") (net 4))
 (segment (start 163.774669 97.87934) (end 164.433678 97.220331) (width 0.25) (layer "F.Cu") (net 4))
 (segment (start 163.774669 99.760331) (end 163.774669 97.87934) (width 0.25) (layer "F.Cu") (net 4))
 (segment (start 164.899669 100.885331) (end 163.774669 99.760331) (width 0.25) (layer "F.Cu") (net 4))
 (segment (start 164.433678 97.220331) (end 175.19 97.220331) (width 0.25) (layer "F.Cu") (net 4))
 (segment (start 176.789669 98.82) (end 179.329669 98.82) (width 0.25) (layer "F.Cu") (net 4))
 (segment (start 166.024669 106.431322) (end 165.23566 107.220331) (width 0.25) (layer "F.Cu") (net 26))
 (segment (start 165.23566 107.220331) (end 138.519669 107.220331) (width 0.25) (layer "F.Cu") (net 26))
 (segment (start 166.024669 104.550331) (end 166.024669 106.431322) (width 0.25) (layer "F.Cu") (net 26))
 (segment (start 138.519669 107.220331) (end 136.859669 105.560331) (width 0.25) (layer "F.Cu") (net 26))
 (segment (start 136.859669 105.560331) (end 136.859669 104.260331) (width 0.25) (layer "F.Cu") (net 26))
 (segment (start 164.899669 103.425331) (end 166.024669 104.550331) (width 0.25) (layer "F.Cu") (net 26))
 (segment (start 163.774669 104.840331) (end 164.899669 105.965331) (width 0.25) (layer "F.Cu") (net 25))
 (segment (start 134.259669 103.135331) (end 134.519669 102.875331) (width 0.25) (layer "F.Cu") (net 25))
 (segment (start 134.259669 104.260331) (end 134.259669 103.135331) (width 0.25) (layer "F.Cu") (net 25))
 (segment (start 134.519669 102.875331) (end 147.85 102.875331) (width 0.25) (layer "F.Cu") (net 25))
 (segment (start 147.85 102.875331) (end 149.815 104.840331) (width 0.25) (layer "F.Cu") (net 25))
 (segment (start 149.815 104.840331) (end 163.774669 104.840331) (width 0.25) (layer "F.Cu") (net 25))
 (segment (start 168.144338 101.59) (end 179.329669 101.59) (width 0.25) (layer "F.Cu") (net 5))
 (segment (start 168.144338 101.59) (end 164.899669 98.345331) (width 0.25) (layer "F.Cu") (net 5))
 (segment (start 134.62 91.44) (end 137.509669 94.329669) (width 0.25) (layer "F.Cu") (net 17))
 (segment (start 137.509669 94.329669) (end 137.509669 97.060331) (width 0.25) (layer "F.Cu") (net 17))
 (segment (start 127 97.79) (end 127 96.52) (width 0.25) (layer "F.Cu") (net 18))
 (segment (start 127 96.52) (end 132.08 91.44) (width 0.25) (layer "F.Cu") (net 18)))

